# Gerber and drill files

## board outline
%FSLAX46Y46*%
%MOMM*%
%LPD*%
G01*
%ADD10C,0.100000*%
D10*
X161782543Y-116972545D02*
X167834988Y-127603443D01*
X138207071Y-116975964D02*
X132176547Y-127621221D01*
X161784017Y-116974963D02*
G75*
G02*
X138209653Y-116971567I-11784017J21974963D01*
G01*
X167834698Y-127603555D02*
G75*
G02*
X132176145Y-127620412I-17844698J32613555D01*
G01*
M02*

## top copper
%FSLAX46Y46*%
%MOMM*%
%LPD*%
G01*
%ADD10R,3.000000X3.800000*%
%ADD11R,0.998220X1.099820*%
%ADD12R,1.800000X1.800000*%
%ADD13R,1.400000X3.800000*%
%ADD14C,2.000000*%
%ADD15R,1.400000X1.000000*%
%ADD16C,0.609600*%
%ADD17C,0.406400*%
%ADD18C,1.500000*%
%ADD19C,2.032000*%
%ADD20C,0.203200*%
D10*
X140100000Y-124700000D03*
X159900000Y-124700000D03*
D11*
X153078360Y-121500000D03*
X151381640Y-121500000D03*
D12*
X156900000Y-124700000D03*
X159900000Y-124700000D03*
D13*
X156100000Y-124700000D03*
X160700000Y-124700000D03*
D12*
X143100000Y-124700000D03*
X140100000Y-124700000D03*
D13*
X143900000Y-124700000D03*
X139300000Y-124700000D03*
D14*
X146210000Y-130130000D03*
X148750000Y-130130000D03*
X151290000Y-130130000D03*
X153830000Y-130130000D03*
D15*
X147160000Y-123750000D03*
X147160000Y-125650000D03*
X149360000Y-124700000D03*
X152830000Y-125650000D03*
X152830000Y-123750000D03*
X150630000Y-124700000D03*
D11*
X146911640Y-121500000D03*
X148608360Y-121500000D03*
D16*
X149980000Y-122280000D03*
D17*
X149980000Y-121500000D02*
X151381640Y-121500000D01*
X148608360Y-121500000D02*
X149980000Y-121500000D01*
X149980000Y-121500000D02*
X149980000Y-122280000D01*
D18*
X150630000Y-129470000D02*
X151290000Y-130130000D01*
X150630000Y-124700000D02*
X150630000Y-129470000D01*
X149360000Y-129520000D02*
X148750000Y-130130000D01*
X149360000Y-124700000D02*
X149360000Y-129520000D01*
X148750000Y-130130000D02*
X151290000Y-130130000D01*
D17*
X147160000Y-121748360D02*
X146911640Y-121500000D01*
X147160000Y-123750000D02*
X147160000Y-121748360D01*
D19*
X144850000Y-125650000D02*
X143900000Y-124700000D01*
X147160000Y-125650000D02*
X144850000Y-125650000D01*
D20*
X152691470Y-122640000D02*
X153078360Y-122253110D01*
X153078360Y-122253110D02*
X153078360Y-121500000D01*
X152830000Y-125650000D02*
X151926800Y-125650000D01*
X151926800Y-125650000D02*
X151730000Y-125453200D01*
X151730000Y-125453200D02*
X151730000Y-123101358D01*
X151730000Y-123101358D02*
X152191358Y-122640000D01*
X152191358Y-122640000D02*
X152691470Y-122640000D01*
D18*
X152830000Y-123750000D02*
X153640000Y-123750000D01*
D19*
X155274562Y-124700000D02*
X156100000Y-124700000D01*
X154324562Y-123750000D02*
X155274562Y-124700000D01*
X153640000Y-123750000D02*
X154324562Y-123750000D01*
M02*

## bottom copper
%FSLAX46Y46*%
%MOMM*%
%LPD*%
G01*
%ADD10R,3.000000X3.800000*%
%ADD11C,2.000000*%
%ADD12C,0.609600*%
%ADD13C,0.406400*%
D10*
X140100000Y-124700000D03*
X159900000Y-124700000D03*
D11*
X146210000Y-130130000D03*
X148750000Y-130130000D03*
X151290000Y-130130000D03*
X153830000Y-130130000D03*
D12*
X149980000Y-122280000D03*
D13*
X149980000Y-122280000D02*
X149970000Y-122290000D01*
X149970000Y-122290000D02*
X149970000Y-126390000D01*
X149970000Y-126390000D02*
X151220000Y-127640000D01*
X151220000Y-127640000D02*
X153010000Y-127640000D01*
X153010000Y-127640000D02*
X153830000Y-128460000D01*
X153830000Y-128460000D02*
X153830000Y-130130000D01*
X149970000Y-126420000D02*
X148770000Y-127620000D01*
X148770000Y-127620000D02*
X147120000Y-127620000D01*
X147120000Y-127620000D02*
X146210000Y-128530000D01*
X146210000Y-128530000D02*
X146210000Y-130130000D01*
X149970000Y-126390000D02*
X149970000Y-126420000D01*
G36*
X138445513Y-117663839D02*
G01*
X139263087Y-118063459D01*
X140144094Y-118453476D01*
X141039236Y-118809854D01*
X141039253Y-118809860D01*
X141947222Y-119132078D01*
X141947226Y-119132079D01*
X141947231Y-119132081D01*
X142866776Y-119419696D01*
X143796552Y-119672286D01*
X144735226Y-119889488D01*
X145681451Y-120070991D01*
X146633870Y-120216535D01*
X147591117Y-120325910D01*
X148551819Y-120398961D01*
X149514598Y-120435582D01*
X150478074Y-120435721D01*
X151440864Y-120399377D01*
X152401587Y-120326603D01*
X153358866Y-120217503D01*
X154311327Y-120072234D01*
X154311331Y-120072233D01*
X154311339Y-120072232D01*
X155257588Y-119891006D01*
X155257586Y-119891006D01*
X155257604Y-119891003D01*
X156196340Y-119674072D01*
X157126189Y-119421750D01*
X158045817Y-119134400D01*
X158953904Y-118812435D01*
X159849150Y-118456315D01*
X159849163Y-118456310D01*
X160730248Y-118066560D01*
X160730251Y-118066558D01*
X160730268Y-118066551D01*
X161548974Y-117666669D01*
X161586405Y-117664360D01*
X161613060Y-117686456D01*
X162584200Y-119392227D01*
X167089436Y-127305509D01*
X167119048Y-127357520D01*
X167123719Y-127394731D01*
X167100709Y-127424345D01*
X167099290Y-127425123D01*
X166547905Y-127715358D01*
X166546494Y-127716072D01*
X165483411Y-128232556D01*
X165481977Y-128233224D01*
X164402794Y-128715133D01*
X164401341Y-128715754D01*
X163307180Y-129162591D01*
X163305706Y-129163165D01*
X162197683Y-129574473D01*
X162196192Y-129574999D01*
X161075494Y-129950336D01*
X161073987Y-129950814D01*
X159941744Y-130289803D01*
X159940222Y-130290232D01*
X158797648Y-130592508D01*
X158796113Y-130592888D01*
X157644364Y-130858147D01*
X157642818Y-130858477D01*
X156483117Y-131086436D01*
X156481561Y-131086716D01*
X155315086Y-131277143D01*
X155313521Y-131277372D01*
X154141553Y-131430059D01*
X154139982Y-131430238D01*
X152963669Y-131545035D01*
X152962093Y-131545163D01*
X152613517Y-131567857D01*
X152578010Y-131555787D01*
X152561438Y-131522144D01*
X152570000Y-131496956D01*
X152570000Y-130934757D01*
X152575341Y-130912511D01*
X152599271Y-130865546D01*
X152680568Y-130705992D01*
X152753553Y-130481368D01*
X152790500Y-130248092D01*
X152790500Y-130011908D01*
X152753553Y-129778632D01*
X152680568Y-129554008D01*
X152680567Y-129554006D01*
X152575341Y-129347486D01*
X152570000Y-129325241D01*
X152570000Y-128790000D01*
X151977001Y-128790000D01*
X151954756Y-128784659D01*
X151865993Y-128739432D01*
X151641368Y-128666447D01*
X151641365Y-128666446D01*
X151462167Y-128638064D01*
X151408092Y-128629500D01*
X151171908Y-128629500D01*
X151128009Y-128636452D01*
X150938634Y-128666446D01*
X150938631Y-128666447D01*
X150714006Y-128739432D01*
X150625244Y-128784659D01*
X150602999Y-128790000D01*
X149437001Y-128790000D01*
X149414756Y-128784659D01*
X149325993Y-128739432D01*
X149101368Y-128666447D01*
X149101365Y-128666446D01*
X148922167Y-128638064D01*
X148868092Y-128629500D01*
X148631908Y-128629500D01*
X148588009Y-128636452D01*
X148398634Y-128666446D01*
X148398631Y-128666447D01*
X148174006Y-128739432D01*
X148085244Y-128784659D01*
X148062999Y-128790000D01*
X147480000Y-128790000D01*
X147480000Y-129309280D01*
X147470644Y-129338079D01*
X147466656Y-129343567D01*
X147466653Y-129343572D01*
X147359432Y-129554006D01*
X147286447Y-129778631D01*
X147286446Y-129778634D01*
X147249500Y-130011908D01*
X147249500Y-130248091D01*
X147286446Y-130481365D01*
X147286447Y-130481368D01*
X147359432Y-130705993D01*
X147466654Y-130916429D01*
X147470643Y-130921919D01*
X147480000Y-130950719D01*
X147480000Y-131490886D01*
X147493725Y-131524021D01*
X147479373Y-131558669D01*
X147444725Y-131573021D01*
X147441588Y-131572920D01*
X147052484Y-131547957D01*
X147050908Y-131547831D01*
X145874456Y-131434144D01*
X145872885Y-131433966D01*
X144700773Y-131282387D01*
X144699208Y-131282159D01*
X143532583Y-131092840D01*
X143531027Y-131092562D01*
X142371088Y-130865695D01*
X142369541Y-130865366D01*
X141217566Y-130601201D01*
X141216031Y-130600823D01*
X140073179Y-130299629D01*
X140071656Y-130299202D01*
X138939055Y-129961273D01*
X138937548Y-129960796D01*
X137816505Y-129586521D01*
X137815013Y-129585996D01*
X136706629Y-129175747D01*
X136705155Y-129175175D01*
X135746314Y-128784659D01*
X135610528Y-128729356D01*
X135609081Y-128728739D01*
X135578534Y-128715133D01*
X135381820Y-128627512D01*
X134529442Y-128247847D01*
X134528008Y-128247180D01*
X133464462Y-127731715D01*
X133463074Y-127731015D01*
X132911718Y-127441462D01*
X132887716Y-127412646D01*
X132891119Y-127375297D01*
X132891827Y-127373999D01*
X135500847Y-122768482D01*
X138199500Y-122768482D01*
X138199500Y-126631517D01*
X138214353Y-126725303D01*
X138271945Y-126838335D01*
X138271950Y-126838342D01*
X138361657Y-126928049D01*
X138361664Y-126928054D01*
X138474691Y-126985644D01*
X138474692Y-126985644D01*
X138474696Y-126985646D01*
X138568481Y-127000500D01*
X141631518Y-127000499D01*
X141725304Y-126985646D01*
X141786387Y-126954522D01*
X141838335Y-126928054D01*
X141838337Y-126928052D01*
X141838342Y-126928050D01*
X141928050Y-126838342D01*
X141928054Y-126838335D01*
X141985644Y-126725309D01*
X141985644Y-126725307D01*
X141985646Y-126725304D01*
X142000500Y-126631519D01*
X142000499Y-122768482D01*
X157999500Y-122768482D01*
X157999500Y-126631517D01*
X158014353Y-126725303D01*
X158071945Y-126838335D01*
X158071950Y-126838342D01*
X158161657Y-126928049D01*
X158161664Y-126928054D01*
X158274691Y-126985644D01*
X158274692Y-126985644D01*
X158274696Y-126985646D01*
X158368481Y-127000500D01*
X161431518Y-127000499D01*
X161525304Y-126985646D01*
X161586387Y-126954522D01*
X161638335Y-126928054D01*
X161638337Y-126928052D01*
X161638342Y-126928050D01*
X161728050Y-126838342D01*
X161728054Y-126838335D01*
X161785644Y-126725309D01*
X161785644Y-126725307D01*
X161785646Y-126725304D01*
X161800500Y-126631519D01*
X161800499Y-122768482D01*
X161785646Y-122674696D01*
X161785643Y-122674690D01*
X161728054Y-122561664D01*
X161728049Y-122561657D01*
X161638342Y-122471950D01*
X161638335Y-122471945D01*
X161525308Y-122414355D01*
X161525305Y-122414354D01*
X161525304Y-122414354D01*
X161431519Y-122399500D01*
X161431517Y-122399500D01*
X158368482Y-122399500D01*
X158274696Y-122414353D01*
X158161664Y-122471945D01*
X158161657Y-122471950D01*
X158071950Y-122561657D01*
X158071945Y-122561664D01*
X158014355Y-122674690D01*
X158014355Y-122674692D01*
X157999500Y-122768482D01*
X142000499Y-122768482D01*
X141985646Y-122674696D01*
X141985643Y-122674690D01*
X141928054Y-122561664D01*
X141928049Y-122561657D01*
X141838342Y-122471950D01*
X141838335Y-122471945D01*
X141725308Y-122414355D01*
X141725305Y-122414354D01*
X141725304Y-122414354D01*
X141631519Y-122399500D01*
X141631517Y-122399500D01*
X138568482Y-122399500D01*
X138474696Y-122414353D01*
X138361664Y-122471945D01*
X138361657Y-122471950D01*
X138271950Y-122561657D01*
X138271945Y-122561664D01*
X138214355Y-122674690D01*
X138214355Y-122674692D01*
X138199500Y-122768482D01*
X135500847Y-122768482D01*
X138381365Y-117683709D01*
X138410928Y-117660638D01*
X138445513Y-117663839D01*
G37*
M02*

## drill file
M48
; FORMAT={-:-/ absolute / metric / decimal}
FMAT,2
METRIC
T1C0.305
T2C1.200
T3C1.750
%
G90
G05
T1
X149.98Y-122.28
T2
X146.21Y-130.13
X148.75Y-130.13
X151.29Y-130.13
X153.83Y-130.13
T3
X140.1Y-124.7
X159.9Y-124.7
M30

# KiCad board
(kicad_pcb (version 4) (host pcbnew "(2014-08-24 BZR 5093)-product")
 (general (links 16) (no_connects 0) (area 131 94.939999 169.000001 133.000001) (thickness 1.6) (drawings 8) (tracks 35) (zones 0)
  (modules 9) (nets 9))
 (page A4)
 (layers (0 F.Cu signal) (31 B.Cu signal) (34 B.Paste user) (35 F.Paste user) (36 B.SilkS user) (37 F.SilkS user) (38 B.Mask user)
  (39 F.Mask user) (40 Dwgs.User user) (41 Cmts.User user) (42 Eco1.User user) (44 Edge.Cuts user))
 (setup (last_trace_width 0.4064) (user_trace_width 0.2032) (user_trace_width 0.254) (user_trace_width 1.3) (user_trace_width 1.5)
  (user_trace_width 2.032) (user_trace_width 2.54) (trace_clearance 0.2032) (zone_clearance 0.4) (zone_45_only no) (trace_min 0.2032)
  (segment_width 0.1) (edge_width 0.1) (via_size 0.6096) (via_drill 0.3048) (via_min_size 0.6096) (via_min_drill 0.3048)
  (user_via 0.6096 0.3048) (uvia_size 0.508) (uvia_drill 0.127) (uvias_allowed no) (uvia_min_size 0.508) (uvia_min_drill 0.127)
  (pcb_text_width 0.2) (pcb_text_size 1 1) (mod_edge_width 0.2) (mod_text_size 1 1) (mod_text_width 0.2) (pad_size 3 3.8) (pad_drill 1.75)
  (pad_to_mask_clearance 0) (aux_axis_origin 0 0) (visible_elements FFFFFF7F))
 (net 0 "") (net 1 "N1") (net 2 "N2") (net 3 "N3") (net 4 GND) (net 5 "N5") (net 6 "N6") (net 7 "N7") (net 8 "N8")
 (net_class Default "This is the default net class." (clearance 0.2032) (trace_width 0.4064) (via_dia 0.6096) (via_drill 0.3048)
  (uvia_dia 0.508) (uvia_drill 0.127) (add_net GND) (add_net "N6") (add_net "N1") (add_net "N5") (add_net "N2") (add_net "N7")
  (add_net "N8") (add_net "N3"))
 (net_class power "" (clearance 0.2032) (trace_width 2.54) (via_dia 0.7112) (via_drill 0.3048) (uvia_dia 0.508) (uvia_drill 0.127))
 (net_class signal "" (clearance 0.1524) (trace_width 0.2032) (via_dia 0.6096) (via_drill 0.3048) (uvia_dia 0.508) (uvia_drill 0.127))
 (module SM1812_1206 (layer B.Cu) (at 141.6 124.7 180) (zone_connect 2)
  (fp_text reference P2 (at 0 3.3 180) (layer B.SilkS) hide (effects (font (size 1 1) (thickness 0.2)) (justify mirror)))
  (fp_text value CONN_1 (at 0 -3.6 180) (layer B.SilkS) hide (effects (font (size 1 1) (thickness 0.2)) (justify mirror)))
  (pad 1 thru_hole rect (at 1.5 0 180) (size 3 3.8) (drill 1.75) (layers *.Cu *.Mask) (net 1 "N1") (zone_connect 2)))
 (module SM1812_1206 (layer B.Cu) (at 158.4 124.7) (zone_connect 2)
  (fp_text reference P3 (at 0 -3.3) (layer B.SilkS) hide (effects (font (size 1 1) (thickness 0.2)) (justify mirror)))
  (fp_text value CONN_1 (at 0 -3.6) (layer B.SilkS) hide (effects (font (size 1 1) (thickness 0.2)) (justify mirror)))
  (pad 1 thru_hole rect (at 1.5 0) (size 3 3.8) (drill 1.75) (layers *.Cu *.Mask) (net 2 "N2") (zone_connect 2)))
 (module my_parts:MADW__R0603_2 (layer F.Cu) (at 152.23 121.5 180)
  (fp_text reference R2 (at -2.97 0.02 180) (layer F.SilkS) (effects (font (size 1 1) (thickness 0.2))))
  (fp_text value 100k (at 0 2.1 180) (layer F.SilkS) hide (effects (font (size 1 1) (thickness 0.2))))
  (pad 1 smd rect (at -0.84836 0 180) (size 0.99822 1.09982) (layers F.Cu F.Paste F.Mask) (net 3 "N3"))
  (pad 2 smd rect (at 0.84836 0 180) (size 0.99822 1.09982) (layers F.Cu F.Paste F.Mask) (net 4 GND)))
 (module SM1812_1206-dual (layer F.Cu) (at 158.4 124.7)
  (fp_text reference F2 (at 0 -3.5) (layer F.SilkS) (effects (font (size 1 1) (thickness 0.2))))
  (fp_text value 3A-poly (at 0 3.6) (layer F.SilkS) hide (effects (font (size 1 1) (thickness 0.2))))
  (pad 1 smd rect (at -1.5 0) (size 1.8 1.8) (layers F.Cu F.Paste F.Mask) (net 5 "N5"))
  (pad 2 smd rect (at 1.5 0) (size 1.8 1.8) (layers F.Cu F.Paste F.Mask) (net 2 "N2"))
  (pad 1 smd rect (at -2.3 0) (size 1.4 3.8) (layers F.Cu F.Paste F.Mask) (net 5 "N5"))
  (pad 2 smd rect (at 2.3 0) (size 1.4 3.8) (layers F.Cu F.Paste F.Mask) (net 2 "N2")))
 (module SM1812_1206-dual (layer F.Cu) (at 141.6 124.7 180)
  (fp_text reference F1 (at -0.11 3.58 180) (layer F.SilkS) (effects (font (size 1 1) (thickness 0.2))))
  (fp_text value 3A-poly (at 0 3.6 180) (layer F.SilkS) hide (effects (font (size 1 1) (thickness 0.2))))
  (pad 1 smd rect (at -1.5 0 180) (size 1.8 1.8) (layers F.Cu F.Paste F.Mask) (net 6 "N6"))
  (pad 2 smd rect (at 1.5 0 180) (size 1.8 1.8) (layers F.Cu F.Paste F.Mask) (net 1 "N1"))
  (pad 1 smd rect (at -2.3 0 180) (size 1.4 3.8) (layers F.Cu F.Paste F.Mask) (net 6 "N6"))
  (pad 2 smd rect (at 2.3 0 180) (size 1.4 3.8) (layers F.Cu F.Paste F.Mask) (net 1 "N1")))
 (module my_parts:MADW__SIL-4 (layer F.Cu) (at 150.02 130.13) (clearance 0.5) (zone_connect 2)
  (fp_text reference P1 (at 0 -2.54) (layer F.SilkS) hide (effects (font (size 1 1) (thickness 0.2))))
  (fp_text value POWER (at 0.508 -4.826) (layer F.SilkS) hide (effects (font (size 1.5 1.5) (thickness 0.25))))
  (pad 1 thru_hole circle (at -3.81 0) (size 2 2) (drill 1.2) (layers *.Cu *.Mask) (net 4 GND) (zone_connect 2))
  (pad 2 thru_hole circle (at -1.27 0) (size 2 2) (drill 1.2) (layers *.Cu *.Mask) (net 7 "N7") (zone_connect 2))
  (pad 3 thru_hole circle (at 1.27 0) (size 2 2) (drill 1.2) (layers *.Cu *.Mask) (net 7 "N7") (zone_connect 2))
  (pad 4 thru_hole circle (at 3.81 0) (size 2 2) (drill 1.2) (layers *.Cu *.Mask) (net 4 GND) (zone_connect 2)))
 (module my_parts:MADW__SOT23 (layer F.Cu) (at 148.26 124.7 270)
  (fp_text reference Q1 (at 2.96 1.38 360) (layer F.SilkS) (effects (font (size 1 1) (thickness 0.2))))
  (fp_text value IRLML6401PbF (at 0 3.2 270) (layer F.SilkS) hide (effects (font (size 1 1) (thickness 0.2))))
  (pad 1 smd rect (at -0.95 1.1 270) (size 1 1.4) (layers F.Cu F.Paste F.Mask) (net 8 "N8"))
  (pad 2 smd rect (at 0.95 1.1 270) (size 1 1.4) (layers F.Cu F.Paste F.Mask) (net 6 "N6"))
  (pad 3 smd rect (at 0 -1.1 270) (size 1 1.4) (layers F.Cu F.Paste F.Mask) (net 7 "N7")))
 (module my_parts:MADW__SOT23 (layer F.Cu) (at 151.73 124.7 90)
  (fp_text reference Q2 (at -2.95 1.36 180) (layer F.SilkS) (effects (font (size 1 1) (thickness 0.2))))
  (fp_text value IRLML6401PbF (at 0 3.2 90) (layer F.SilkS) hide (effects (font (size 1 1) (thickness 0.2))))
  (pad 1 smd rect (at -0.95 1.1 90) (size 1 1.4) (layers F.Cu F.Paste F.Mask) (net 3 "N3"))
  (pad 2 smd rect (at 0.95 1.1 90) (size 1 1.4) (layers F.Cu F.Paste F.Mask) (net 5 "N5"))
  (pad 3 smd rect (at 0 -1.1 90) (size 1 1.4) (layers F.Cu F.Paste F.Mask) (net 7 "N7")))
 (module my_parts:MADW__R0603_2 (layer F.Cu) (at 147.76 121.5)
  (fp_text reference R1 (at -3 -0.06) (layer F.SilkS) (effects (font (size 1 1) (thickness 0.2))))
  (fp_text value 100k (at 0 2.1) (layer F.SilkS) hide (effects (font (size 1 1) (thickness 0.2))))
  (pad 1 smd rect (at -0.84836 0) (size 0.99822 1.09982) (layers F.Cu F.Paste F.Mask) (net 8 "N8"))
  (pad 2 smd rect (at 0.84836 0) (size 0.99822 1.09982) (layers F.Cu F.Paste F.Mask) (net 4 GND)))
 (gr_line (start 161.782543 116.972545) (end 167.834988 127.603443) (layer Edge.Cuts) (width 0.1))
 (gr_line (start 138.207071 116.975964) (end 132.176547 127.621221) (layer Edge.Cuts) (width 0.1))
 (gr_arc (start 150 95) (end 161.784017 116.974963) (angle 56.42114376) (layer Edge.Cuts) (width 0.1))
 (gr_arc (start 149.99 94.99) (end 167.834698 127.603555) (angle 57.316895) (layer Edge.Cuts) (width 0.1))
 (segment (start 149.98 122.28) (end 149.97 122.29) (width 0.4064) (layer B.Cu) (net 4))
 (segment (start 149.97 122.29) (end 149.97 126.39) (width 0.4064) (layer B.Cu) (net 4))
 (segment (start 149.97 126.39) (end 151.22 127.64) (width 0.4064) (layer B.Cu) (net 4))
 (segment (start 151.22 127.64) (end 153.01 127.64) (width 0.4064) (layer B.Cu) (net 4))
 (segment (start 153.01 127.64) (end 153.83 128.46) (width 0.4064) (layer B.Cu) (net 4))
 (segment (start 153.83 128.46) (end 153.83 130.13) (width 0.4064) (layer B.Cu) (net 4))
 (segment (start 149.97 126.42) (end 148.77 127.62) (width 0.4064) (layer B.Cu) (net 4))
 (segment (start 148.77 127.62) (end 147.12 127.62) (width 0.4064) (layer B.Cu) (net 4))
 (segment (start 147.12 127.62) (end 146.21 128.53) (width 0.4064) (layer B.Cu) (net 4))
 (segment (start 146.21 128.53) (end 146.21 130.13) (width 0.4064) (layer B.Cu) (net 4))
 (segment (start 149.97 126.39) (end 149.97 126.42) (width 0.4064) (layer B.Cu) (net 4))
 (segment (start 149.98 121.5) (end 151.38164 121.5) (width 0.4064) (layer F.Cu) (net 4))
 (segment (start 148.60836 121.5) (end 149.98 121.5) (width 0.4064) (layer F.Cu) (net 4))
 (via (at 149.98 122.28) (size 0.6096) (layers F.Cu B.Cu) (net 4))
 (segment (start 149.98 121.5) (end 149.98 122.28) (width 0.4064) (layer F.Cu) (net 4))
 (segment (start 150.63 129.47) (end 151.29 130.13) (width 1.5) (layer F.Cu) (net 7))
 (segment (start 150.63 124.7) (end 150.63 129.47) (width 1.5) (layer F.Cu) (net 7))
 (segment (start 149.36 129.52) (end 148.75 130.13) (width 1.5) (layer F.Cu) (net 7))
 (segment (start 149.36 124.7) (end 149.36 129.52) (width 1.5) (layer F.Cu) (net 7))
 (segment (start 148.75 130.13) (end 151.29 130.13) (width 1.5) (layer F.Cu) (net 7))
 (segment (start 147.16 121.74836) (end 146.91164 121.5) (width 0.4064) (layer F.Cu) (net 8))
 (segment (start 147.16 123.75) (end 147.16 121.74836) (width 0.4064) (layer F.Cu) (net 8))
 (segment (start 144.85 125.65) (end 143.9 124.7) (width 2.032) (layer F.Cu) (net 6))
 (segment (start 147.16 125.65) (end 144.85 125.65) (width 2.032) (layer F.Cu) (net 6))
 (segment (start 152.69147 122.64) (end 153.07836 122.25311) (width 0.2032) (layer F.Cu) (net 3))
 (segment (start 153.07836 122.25311) (end 153.07836 121.5) (width 0.2032) (layer F.Cu) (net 3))
 (segment (start 152.83 125.65) (end 151.9268 125.65) (width 0.2032) (layer F.Cu) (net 3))
 (segment (start 151.9268 125.65) (end 151.73 125.4532) (width 0.2032) (layer F.Cu) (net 3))
 (segment (start 151.73 125.4532) (end 151.73 123.101358) (width 0.2032) (layer F.Cu) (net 3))
 (segment (start 151.73 123.101358) (end 152.191358 122.64) (width 0.2032) (layer F.Cu) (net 3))
 (segment (start 152.191358 122.64) (end 152.69147 122.64) (width 0.2032) (layer F.Cu) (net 3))
 (segment (start 152.83 123.75) (end 153.64 123.75) (width 1.5) (layer F.Cu) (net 5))
 (segment (start 155.274562 124.7) (end 156.1 124.7) (width 2.032) (layer F.Cu) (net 5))
 (segment (start 154.324562 123.75) (end 155.274562 124.7) (width 2.032) (layer F.Cu) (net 5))
 (segment (start 153.64 123.75) (end 154.324562 123.75) (width 2.032) (layer F.Cu) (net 5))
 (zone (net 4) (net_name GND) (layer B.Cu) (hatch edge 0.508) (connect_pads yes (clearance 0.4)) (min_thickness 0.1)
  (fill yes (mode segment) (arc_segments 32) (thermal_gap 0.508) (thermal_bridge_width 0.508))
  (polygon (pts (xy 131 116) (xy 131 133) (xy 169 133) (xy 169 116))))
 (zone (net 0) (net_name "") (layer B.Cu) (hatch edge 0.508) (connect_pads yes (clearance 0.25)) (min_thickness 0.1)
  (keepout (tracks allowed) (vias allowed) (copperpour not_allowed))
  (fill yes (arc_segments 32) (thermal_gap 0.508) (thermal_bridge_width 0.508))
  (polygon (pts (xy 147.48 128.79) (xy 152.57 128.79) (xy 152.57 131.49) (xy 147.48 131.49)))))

